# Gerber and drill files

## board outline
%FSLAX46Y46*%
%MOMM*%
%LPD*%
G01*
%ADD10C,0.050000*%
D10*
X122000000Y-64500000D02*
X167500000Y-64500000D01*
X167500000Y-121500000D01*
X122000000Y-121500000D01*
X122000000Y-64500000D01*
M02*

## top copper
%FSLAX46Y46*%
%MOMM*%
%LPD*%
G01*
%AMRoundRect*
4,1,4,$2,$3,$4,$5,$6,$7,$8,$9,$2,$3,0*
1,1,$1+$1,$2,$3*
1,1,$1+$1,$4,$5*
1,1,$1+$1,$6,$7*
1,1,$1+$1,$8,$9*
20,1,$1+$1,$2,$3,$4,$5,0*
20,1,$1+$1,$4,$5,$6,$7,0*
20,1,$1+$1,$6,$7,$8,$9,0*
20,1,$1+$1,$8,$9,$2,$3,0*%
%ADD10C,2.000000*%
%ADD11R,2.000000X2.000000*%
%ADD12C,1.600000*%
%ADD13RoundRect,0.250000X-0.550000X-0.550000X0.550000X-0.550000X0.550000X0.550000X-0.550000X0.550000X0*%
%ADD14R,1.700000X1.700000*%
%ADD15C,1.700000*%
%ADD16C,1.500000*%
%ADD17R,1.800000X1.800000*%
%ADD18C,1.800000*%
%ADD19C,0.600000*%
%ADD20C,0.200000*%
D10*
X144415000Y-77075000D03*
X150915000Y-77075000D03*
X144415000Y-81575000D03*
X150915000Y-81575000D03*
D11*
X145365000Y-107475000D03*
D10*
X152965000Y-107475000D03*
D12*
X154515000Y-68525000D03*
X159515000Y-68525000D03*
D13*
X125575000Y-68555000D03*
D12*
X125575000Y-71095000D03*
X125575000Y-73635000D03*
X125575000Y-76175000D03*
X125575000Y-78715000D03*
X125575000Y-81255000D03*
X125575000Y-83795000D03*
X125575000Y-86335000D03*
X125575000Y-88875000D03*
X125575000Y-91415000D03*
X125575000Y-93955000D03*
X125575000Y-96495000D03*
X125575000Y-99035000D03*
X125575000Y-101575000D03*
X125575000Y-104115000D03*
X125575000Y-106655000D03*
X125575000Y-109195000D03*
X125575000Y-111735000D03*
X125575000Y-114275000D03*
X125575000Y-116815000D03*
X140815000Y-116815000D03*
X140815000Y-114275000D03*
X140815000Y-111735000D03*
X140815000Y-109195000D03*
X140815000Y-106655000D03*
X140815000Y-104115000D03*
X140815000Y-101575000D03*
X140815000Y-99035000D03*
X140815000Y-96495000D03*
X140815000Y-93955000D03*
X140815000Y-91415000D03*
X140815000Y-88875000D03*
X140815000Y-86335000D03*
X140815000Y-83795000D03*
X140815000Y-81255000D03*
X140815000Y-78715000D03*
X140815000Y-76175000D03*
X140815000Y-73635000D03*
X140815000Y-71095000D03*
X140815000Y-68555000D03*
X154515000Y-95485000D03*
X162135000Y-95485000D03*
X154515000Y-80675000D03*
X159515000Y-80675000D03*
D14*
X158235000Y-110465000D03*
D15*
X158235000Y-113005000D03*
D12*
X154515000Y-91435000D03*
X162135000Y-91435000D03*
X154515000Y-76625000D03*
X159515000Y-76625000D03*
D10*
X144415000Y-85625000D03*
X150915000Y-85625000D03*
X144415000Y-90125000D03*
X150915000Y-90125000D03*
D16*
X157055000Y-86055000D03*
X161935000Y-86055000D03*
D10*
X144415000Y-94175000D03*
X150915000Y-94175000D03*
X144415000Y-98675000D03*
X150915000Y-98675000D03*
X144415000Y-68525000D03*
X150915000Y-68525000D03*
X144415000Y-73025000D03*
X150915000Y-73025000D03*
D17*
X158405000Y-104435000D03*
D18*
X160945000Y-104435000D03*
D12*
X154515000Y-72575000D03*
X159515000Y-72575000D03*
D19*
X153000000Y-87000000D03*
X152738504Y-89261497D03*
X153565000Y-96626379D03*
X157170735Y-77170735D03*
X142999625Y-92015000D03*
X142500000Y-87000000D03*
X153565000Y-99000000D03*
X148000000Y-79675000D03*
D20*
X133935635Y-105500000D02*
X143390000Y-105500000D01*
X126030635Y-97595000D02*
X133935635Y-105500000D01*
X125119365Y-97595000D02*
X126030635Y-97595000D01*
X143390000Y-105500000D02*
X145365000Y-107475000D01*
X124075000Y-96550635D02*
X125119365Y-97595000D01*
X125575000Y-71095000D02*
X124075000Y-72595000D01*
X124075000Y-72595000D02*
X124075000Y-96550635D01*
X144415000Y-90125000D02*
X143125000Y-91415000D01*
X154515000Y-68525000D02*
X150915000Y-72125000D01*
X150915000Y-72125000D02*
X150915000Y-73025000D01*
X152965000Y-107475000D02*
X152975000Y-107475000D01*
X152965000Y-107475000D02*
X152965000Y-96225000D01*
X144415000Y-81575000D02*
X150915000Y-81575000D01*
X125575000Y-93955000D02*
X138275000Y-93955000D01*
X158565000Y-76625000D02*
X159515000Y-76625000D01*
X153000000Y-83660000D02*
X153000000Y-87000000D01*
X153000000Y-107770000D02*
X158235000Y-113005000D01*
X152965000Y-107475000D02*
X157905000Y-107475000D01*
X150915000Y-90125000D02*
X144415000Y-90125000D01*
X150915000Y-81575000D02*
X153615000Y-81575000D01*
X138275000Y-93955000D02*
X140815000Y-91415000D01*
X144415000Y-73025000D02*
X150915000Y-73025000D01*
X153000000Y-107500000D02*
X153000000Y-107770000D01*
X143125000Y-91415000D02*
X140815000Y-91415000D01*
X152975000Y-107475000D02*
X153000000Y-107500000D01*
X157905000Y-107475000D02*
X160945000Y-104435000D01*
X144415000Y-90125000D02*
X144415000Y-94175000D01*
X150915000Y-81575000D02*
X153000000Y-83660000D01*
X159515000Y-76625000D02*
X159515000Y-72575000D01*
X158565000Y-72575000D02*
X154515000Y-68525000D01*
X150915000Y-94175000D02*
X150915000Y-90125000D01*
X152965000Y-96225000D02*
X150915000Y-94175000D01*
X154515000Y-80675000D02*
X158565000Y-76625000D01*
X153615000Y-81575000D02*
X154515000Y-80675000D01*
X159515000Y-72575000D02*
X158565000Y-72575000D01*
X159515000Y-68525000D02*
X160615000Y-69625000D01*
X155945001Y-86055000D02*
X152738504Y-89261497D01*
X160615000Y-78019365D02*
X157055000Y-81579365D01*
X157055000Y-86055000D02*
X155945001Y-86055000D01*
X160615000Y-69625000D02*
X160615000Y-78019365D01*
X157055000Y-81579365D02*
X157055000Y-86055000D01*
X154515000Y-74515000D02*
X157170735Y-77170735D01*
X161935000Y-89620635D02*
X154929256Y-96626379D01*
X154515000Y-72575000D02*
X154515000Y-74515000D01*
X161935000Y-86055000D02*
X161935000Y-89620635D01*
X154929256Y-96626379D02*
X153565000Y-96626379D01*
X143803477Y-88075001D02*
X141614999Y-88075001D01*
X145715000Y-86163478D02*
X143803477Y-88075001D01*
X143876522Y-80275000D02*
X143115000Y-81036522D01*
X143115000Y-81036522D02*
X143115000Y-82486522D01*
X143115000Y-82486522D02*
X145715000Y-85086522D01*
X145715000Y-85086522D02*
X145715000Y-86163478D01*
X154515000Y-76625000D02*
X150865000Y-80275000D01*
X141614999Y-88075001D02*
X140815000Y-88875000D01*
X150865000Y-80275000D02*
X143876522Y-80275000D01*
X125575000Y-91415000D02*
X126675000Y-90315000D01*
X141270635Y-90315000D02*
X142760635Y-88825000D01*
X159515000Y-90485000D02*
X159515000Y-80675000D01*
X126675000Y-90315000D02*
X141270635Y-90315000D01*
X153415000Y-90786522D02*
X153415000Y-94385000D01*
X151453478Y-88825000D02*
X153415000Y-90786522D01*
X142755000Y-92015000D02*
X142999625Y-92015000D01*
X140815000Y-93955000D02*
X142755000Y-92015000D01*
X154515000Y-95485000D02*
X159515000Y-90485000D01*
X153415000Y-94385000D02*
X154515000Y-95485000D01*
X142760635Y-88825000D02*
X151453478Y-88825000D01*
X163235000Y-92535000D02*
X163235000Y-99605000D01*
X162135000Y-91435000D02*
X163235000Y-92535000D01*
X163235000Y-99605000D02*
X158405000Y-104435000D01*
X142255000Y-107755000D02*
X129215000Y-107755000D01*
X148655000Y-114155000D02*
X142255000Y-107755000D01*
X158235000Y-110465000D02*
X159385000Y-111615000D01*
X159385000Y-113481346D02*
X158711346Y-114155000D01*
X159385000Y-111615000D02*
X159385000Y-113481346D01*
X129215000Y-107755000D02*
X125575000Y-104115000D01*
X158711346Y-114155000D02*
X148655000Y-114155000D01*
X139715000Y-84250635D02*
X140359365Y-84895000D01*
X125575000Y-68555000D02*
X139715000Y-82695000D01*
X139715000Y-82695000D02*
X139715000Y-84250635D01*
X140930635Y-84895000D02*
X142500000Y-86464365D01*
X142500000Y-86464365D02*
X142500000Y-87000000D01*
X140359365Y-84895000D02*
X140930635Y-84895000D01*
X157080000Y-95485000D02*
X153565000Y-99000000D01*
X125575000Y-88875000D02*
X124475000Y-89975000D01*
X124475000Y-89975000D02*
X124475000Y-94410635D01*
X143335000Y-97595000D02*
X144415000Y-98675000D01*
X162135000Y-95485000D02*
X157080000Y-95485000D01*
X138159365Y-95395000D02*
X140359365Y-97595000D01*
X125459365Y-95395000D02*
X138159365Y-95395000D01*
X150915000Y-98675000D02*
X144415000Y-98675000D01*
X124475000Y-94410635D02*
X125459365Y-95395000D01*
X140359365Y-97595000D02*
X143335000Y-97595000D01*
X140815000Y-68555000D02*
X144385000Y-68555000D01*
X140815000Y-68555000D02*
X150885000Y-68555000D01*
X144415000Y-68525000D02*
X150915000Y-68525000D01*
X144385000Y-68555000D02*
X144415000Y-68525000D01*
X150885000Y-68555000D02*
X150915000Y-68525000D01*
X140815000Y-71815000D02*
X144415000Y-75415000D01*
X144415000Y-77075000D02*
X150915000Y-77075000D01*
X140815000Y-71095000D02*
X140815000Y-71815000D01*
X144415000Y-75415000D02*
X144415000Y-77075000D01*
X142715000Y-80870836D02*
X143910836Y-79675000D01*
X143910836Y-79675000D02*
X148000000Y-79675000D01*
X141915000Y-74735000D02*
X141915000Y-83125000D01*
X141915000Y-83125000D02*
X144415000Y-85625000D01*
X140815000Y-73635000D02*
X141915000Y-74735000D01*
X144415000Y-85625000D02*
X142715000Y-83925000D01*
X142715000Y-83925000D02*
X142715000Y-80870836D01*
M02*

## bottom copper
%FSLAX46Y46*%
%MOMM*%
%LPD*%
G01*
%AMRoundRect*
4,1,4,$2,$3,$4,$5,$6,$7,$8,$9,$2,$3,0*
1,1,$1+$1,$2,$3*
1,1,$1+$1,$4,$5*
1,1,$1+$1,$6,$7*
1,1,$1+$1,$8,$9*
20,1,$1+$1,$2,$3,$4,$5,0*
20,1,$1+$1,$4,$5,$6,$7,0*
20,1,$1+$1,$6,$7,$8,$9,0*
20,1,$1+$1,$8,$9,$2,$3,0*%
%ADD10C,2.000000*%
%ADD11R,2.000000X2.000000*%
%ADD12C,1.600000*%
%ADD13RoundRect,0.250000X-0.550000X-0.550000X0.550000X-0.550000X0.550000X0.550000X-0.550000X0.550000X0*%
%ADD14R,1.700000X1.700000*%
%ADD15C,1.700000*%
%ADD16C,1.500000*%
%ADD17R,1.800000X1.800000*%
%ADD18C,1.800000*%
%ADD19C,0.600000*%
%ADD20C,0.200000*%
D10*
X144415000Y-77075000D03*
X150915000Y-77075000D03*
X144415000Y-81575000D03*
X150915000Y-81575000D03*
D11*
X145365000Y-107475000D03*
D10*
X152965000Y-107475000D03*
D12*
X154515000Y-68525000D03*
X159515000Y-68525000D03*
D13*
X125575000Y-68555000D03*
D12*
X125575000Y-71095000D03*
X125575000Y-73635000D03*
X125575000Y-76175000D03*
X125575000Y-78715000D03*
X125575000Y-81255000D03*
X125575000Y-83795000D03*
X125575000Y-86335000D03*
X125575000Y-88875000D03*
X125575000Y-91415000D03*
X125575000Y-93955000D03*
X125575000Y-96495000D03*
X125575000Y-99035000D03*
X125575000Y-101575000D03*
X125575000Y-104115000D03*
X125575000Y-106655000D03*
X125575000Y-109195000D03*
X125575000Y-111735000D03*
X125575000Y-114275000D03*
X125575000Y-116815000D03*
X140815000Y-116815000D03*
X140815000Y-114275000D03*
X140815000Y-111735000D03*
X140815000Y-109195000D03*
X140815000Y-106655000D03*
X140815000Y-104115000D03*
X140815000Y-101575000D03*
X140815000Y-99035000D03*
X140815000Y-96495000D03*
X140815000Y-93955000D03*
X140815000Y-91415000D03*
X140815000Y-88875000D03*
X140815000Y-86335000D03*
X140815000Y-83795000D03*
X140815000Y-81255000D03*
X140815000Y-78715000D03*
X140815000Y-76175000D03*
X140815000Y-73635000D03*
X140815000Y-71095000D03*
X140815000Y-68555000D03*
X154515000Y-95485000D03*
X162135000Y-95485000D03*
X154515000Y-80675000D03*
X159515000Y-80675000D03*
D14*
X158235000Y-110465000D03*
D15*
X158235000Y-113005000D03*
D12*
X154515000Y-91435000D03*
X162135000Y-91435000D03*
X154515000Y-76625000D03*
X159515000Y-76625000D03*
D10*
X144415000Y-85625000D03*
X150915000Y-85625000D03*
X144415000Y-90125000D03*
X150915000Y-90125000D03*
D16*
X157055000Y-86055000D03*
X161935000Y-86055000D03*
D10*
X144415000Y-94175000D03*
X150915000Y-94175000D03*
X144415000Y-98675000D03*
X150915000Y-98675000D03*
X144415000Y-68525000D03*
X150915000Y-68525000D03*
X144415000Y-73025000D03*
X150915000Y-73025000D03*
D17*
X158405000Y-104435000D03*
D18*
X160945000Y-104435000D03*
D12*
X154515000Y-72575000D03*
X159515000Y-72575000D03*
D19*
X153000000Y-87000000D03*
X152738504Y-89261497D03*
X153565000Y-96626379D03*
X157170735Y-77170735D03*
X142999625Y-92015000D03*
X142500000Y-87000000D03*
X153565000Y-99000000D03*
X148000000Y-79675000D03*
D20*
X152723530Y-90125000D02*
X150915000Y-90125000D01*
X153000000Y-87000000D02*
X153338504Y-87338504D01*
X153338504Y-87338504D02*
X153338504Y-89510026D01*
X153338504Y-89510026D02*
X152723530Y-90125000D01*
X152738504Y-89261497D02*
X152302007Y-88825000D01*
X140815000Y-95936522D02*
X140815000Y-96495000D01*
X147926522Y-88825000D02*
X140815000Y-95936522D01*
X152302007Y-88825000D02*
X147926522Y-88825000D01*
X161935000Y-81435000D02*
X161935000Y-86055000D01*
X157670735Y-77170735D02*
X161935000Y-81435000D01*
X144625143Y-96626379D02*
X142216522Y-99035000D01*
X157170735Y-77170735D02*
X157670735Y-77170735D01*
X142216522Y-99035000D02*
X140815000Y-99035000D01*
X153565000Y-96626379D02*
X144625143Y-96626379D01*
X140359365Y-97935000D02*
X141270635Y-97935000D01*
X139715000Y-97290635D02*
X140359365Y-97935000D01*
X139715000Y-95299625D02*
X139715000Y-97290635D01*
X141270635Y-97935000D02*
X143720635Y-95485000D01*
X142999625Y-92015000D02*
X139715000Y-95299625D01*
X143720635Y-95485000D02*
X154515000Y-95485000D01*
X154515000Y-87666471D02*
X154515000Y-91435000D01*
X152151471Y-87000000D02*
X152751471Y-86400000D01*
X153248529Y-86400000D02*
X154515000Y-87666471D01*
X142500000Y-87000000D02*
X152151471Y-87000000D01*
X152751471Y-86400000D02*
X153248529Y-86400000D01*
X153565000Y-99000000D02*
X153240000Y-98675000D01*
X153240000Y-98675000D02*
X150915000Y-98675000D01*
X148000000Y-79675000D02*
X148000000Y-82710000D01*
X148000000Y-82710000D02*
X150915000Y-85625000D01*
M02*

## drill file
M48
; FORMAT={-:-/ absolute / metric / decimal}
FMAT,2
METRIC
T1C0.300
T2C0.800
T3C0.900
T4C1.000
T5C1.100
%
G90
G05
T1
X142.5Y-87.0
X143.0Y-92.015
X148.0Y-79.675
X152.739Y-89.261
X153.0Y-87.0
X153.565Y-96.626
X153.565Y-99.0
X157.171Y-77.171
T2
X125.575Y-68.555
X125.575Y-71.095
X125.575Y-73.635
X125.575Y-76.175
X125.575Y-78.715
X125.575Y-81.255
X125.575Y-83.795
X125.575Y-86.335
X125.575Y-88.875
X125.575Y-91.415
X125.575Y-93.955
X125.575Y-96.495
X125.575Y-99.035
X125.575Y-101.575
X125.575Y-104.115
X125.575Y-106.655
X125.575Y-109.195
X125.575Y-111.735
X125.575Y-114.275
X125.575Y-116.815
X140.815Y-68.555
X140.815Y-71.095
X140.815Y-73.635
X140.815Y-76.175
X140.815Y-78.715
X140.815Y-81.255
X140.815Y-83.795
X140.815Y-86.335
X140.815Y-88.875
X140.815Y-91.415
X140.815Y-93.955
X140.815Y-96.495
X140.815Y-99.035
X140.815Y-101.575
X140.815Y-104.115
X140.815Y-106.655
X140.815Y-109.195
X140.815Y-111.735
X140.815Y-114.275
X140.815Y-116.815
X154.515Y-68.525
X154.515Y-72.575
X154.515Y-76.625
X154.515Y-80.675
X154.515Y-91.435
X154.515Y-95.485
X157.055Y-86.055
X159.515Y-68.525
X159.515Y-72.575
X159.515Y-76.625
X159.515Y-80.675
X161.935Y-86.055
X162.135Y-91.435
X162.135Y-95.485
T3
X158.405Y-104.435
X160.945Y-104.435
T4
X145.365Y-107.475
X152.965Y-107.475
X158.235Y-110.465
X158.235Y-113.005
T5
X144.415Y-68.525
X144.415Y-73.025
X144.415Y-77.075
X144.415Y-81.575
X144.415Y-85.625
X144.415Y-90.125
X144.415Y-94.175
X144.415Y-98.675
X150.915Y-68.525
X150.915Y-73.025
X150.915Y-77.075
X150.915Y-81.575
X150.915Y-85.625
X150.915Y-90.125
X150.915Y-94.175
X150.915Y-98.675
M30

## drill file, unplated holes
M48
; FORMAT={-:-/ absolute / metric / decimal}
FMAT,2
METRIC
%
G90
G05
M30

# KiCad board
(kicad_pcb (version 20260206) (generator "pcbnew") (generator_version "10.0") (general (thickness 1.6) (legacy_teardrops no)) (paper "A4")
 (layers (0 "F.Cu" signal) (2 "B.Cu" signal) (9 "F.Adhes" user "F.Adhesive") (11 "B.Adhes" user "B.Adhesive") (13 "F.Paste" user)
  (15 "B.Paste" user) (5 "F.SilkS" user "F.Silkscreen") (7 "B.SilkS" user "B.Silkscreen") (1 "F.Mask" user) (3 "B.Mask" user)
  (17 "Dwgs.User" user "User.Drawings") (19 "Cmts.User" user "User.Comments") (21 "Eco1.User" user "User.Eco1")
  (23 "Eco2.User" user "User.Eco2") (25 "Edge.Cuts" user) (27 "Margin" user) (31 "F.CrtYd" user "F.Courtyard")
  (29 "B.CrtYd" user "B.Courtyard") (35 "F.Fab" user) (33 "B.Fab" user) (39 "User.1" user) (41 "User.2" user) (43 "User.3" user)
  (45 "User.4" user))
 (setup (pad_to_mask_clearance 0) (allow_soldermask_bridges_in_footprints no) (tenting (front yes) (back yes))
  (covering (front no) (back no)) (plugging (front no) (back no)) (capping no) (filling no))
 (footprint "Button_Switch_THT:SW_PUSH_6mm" (layer "F.Cu") (at 144.415 77.075)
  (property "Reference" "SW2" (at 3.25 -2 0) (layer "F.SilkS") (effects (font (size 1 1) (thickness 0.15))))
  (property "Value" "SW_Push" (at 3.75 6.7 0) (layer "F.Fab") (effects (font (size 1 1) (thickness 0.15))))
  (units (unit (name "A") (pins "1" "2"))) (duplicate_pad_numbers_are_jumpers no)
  (pad "1" thru_hole circle (at 0 0 90) (size 2 2) (drill 1.1) (layers "*.Cu" "*.Mask") (remove_unused_layers no) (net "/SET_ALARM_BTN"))
  (pad "1" thru_hole circle (at 6.5 0 90) (size 2 2) (drill 1.1) (layers "*.Cu" "*.Mask") (remove_unused_layers no) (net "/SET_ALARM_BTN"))
  (pad "2" thru_hole circle (at 0 4.5 90) (size 2 2) (drill 1.1) (layers "*.Cu" "*.Mask") (remove_unused_layers no) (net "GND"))
  (pad "2" thru_hole circle (at 6.5 4.5 90) (size 2 2) (drill 1.1) (layers "*.Cu" "*.Mask") (remove_unused_layers no) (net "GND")))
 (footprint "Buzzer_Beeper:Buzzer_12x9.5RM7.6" (layer "F.Cu") (at 145.365 107.475)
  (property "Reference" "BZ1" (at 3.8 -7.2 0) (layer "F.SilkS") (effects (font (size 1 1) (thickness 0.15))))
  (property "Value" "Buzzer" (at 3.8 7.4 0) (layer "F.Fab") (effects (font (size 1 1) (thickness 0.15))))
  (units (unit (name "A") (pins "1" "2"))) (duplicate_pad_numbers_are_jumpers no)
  (pad "1" thru_hole rect (at 0 0) (size 2 2) (drill 1) (layers "*.Cu" "*.Mask") (remove_unused_layers no) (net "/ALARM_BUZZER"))
  (pad "2" thru_hole circle (at 7.6 0) (size 2 2) (drill 1) (layers "*.Cu" "*.Mask") (remove_unused_layers no) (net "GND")))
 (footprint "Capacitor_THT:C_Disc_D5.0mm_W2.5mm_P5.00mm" (layer "F.Cu") (at 154.515 68.525)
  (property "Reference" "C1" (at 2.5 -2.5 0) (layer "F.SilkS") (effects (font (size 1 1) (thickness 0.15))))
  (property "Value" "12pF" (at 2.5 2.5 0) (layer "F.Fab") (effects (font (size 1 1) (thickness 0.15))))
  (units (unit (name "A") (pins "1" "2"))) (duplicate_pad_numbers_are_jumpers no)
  (pad "1" thru_hole circle (at 0 0) (size 1.6 1.6) (drill 0.8) (layers "*.Cu" "*.Mask") (remove_unused_layers no) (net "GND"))
  (pad "2" thru_hole circle (at 5 0) (size 1.6 1.6) (drill 0.8) (layers "*.Cu" "*.Mask") (remove_unused_layers no) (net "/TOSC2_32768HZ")))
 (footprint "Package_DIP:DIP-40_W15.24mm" (layer "F.Cu") (at 125.575 68.555)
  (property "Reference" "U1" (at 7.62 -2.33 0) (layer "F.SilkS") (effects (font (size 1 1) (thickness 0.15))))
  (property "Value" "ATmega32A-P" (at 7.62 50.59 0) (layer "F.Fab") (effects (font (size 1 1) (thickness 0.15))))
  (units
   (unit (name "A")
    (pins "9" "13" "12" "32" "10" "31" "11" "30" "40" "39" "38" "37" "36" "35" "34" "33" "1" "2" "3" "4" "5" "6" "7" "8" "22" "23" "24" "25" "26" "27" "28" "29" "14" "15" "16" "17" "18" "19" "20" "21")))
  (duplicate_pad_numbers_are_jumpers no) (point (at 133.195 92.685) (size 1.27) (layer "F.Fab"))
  (pad "1" thru_hole roundrect (at 0 0) (size 1.6 1.6) (drill 0.8) (layers "*.Cu" "*.Mask") (remove_unused_layers no)
   (roundrect_rratio 0.15625) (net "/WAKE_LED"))
  (pad "2" thru_hole circle (at 0 2.54) (size 1.6 1.6) (drill 0.8) (layers "*.Cu" "*.Mask") (remove_unused_layers no) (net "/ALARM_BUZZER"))
  (pad "3" thru_hole circle (at 0 5.08) (size 1.6 1.6) (drill 0.8) (layers "*.Cu" "*.Mask") (remove_unused_layers no)
   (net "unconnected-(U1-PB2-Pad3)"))
  (pad "4" thru_hole circle (at 0 7.62) (size 1.6 1.6) (drill 0.8) (layers "*.Cu" "*.Mask") (remove_unused_layers no)
   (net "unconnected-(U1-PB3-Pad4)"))
  (pad "5" thru_hole circle (at 0 10.16) (size 1.6 1.6) (drill 0.8) (layers "*.Cu" "*.Mask") (remove_unused_layers no)
   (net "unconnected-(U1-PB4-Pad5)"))
  (pad "6" thru_hole circle (at 0 12.7) (size 1.6 1.6) (drill 0.8) (layers "*.Cu" "*.Mask") (remove_unused_layers no)
   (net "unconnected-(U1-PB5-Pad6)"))
  (pad "7" thru_hole circle (at 0 15.24) (size 1.6 1.6) (drill 0.8) (layers "*.Cu" "*.Mask") (remove_unused_layers no)
   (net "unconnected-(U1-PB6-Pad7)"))
  (pad "8" thru_hole circle (at 0 17.78) (size 1.6 1.6) (drill 0.8) (layers "*.Cu" "*.Mask") (remove_unused_layers no)
   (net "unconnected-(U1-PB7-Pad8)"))
  (pad "9" thru_hole circle (at 0 20.32) (size 1.6 1.6) (drill 0.8) (layers "*.Cu" "*.Mask") (remove_unused_layers no)
   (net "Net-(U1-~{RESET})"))
  (pad "10" thru_hole circle (at 0 22.86) (size 1.6 1.6) (drill 0.8) (layers "*.Cu" "*.Mask") (remove_unused_layers no) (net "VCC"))
  (pad "11" thru_hole circle (at 0 25.4) (size 1.6 1.6) (drill 0.8) (layers "*.Cu" "*.Mask") (remove_unused_layers no) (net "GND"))
  (pad "12" thru_hole circle (at 0 27.94) (size 1.6 1.6) (drill 0.8) (layers "*.Cu" "*.Mask") (remove_unused_layers no)
   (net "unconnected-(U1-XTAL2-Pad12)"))
  (pad "13" thru_hole circle (at 0 30.48) (size 1.6 1.6) (drill 0.8) (layers "*.Cu" "*.Mask") (remove_unused_layers no)
   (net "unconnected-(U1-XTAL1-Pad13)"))
  (pad "14" thru_hole circle (at 0 33.02) (size 1.6 1.6) (drill 0.8) (layers "*.Cu" "*.Mask") (remove_unused_layers no)
   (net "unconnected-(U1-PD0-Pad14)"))
  (pad "15" thru_hole circle (at 0 35.56) (size 1.6 1.6) (drill 0.8) (layers "*.Cu" "*.Mask") (remove_unused_layers no)
   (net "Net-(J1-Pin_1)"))
  (pad "16" thru_hole circle (at 0 38.1) (size 1.6 1.6) (drill 0.8) (layers "*.Cu" "*.Mask") (remove_unused_layers no)
   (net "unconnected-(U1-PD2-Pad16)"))
  (pad "17" thru_hole circle (at 0 40.64) (size 1.6 1.6) (drill 0.8) (layers "*.Cu" "*.Mask") (remove_unused_layers no)
   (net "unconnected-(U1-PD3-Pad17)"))
  (pad "18" thru_hole circle (at 0 43.18) (size 1.6 1.6) (drill 0.8) (layers "*.Cu" "*.Mask") (remove_unused_layers no)
   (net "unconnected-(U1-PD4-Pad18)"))
  (pad "19" thru_hole circle (at 0 45.72) (size 1.6 1.6) (drill 0.8) (layers "*.Cu" "*.Mask") (remove_unused_layers no)
   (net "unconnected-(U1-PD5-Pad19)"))
  (pad "20" thru_hole circle (at 0 48.26) (size 1.6 1.6) (drill 0.8) (layers "*.Cu" "*.Mask") (remove_unused_layers no)
   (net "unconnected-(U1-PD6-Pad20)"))
  (pad "21" thru_hole circle (at 15.24 48.26) (size 1.6 1.6) (drill 0.8) (layers "*.Cu" "*.Mask") (remove_unused_layers no)
   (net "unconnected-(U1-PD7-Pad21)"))
  (pad "22" thru_hole circle (at 15.24 45.72) (size 1.6 1.6) (drill 0.8) (layers "*.Cu" "*.Mask") (remove_unused_layers no)
   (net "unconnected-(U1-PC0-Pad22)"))
  (pad "23" thru_hole circle (at 15.24 43.18) (size 1.6 1.6) (drill 0.8) (layers "*.Cu" "*.Mask") (remove_unused_layers no)
   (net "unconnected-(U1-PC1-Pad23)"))
  (pad "24" thru_hole circle (at 15.24 40.64) (size 1.6 1.6) (drill 0.8) (layers "*.Cu" "*.Mask") (remove_unused_layers no)
   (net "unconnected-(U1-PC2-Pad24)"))
  (pad "25" thru_hole circle (at 15.24 38.1) (size 1.6 1.6) (drill 0.8) (layers "*.Cu" "*.Mask") (remove_unused_layers no)
   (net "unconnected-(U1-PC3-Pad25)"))
  (pad "26" thru_hole circle (at 15.24 35.56) (size 1.6 1.6) (drill 0.8) (layers "*.Cu" "*.Mask") (remove_unused_layers no)
   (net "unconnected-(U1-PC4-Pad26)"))
  (pad "27" thru_hole circle (at 15.24 33.02) (size 1.6 1.6) (drill 0.8) (layers "*.Cu" "*.Mask") (remove_unused_layers no)
   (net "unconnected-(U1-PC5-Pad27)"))
  (pad "28" thru_hole circle (at 15.24 30.48) (size 1.6 1.6) (drill 0.8) (layers "*.Cu" "*.Mask") (remove_unused_layers no)
   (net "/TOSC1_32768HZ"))
  (pad "29" thru_hole circle (at 15.24 27.94) (size 1.6 1.6) (drill 0.8) (layers "*.Cu" "*.Mask") (remove_unused_layers no)
   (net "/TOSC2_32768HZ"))
  (pad "30" thru_hole circle (at 15.24 25.4) (size 1.6 1.6) (drill 0.8) (layers "*.Cu" "*.Mask") (remove_unused_layers no) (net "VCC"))
  (pad "31" thru_hole circle (at 15.24 22.86) (size 1.6 1.6) (drill 0.8) (layers "*.Cu" "*.Mask") (remove_unused_layers no) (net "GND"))
  (pad "32" thru_hole circle (at 15.24 20.32) (size 1.6 1.6) (drill 0.8) (layers "*.Cu" "*.Mask") (remove_unused_layers no)
   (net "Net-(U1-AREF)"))
  (pad "33" thru_hole circle (at 15.24 17.78) (size 1.6 1.6) (drill 0.8) (layers "*.Cu" "*.Mask") (remove_unused_layers no)
   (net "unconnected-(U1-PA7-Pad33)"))
  (pad "34" thru_hole circle (at 15.24 15.24) (size 1.6 1.6) (drill 0.8) (layers "*.Cu" "*.Mask") (remove_unused_layers no)
   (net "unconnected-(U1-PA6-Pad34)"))
  (pad "35" thru_hole circle (at 15.24 12.7) (size 1.6 1.6) (drill 0.8) (layers "*.Cu" "*.Mask") (remove_unused_layers no)
   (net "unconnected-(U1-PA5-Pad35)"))
  (pad "36" thru_hole circle (at 15.24 10.16) (size 1.6 1.6) (drill 0.8) (layers "*.Cu" "*.Mask") (remove_unused_layers no)
   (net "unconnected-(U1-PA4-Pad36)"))
  (pad "37" thru_hole circle (at 15.24 7.62) (size 1.6 1.6) (drill 0.8) (layers "*.Cu" "*.Mask") (remove_unused_layers no)
   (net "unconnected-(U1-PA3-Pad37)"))
  (pad "38" thru_hole circle (at 15.24 5.08) (size 1.6 1.6) (drill 0.8) (layers "*.Cu" "*.Mask") (remove_unused_layers no)
   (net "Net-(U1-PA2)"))
  (pad "39" thru_hole circle (at 15.24 2.54) (size 1.6 1.6) (drill 0.8) (layers "*.Cu" "*.Mask") (remove_unused_layers no)
   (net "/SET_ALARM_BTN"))
  (pad "40" thru_hole circle (at 15.24 0) (size 1.6 1.6) (drill 0.8) (layers "*.Cu" "*.Mask") (remove_unused_layers no) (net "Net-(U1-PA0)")))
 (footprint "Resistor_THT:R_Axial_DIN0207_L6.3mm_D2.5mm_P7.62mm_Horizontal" (layer "F.Cu") (at 154.515 95.485)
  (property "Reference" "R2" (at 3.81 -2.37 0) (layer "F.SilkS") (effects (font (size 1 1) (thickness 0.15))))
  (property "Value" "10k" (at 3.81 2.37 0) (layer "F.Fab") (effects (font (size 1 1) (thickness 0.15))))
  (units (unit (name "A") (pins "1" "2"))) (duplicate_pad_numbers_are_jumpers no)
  (pad "1" thru_hole circle (at 0 0) (size 1.6 1.6) (drill 0.8) (layers "*.Cu" "*.Mask") (remove_unused_layers no) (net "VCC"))
  (pad "2" thru_hole circle (at 7.62 0) (size 1.6 1.6) (drill 0.8) (layers "*.Cu" "*.Mask") (remove_unused_layers no)
   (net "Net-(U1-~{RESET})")))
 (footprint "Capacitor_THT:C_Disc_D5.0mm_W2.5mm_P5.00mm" (layer "F.Cu") (at 154.515 80.675)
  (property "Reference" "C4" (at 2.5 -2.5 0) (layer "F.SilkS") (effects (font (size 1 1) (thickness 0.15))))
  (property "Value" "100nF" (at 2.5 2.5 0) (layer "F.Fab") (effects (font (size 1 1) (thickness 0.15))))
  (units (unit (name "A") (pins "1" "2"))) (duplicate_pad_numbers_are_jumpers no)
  (pad "1" thru_hole circle (at 0 0) (size 1.6 1.6) (drill 0.8) (layers "*.Cu" "*.Mask") (remove_unused_layers no) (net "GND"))
  (pad "2" thru_hole circle (at 5 0) (size 1.6 1.6) (drill 0.8) (layers "*.Cu" "*.Mask") (remove_unused_layers no) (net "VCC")))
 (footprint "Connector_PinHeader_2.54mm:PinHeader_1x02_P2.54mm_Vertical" (layer "F.Cu") (at 158.235 110.465)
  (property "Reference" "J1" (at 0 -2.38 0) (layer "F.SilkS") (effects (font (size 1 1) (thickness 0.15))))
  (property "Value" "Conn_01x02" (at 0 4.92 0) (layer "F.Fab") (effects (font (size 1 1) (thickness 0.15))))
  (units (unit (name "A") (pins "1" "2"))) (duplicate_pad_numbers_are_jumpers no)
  (pad "1" thru_hole rect (at 0 0) (size 1.7 1.7) (drill 1) (layers "*.Cu" "*.Mask") (remove_unused_layers no) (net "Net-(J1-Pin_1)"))
  (pad "2" thru_hole circle (at 0 2.54) (size 1.7 1.7) (drill 1) (layers "*.Cu" "*.Mask") (remove_unused_layers no) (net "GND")))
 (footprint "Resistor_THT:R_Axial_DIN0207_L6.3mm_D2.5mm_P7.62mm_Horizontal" (layer "F.Cu") (at 154.515 91.435)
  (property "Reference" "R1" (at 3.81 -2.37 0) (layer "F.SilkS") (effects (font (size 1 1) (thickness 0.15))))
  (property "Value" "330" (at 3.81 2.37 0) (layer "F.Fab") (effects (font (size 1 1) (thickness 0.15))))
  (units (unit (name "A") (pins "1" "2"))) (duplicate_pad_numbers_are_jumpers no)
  (pad "1" thru_hole circle (at 0 0) (size 1.6 1.6) (drill 0.8) (layers "*.Cu" "*.Mask") (remove_unused_layers no) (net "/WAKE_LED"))
  (pad "2" thru_hole circle (at 7.62 0) (size 1.6 1.6) (drill 0.8) (layers "*.Cu" "*.Mask") (remove_unused_layers no) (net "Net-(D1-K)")))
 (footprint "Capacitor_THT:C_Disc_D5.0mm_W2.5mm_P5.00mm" (layer "F.Cu") (at 154.515 76.625)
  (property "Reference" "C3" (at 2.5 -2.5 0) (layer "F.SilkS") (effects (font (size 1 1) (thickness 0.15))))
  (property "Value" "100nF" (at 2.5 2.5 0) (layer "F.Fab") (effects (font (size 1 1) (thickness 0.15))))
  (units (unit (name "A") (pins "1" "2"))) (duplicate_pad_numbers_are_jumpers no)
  (pad "1" thru_hole circle (at 0 0) (size 1.6 1.6) (drill 0.8) (layers "*.Cu" "*.Mask") (remove_unused_layers no) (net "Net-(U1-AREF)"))
  (pad "2" thru_hole circle (at 5 0) (size 1.6 1.6) (drill 0.8) (layers "*.Cu" "*.Mask") (remove_unused_layers no) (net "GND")))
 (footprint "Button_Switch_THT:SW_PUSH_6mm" (layer "F.Cu") (at 144.415 85.625)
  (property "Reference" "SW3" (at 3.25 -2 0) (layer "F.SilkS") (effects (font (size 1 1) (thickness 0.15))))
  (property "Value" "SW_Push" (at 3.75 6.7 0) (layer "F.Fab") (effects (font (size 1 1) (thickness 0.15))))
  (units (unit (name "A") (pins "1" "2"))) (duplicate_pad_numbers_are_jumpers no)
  (pad "1" thru_hole circle (at 0 0 90) (size 2 2) (drill 1.1) (layers "*.Cu" "*.Mask") (remove_unused_layers no) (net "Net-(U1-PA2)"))
  (pad "1" thru_hole circle (at 6.5 0 90) (size 2 2) (drill 1.1) (layers "*.Cu" "*.Mask") (remove_unused_layers no) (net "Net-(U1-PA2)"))
  (pad "2" thru_hole circle (at 0 4.5 90) (size 2 2) (drill 1.1) (layers "*.Cu" "*.Mask") (remove_unused_layers no) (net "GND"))
  (pad "2" thru_hole circle (at 6.5 4.5 90) (size 2 2) (drill 1.1) (layers "*.Cu" "*.Mask") (remove_unused_layers no) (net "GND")))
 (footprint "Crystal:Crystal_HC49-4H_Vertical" (layer "F.Cu") (at 157.055 86.055)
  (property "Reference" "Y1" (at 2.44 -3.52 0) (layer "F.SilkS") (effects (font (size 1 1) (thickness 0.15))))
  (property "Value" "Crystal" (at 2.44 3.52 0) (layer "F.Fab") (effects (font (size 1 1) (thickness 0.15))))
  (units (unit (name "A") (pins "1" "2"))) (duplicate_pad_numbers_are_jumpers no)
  (pad "1" thru_hole circle (at 0 0) (size 1.5 1.5) (drill 0.8) (layers "*.Cu" "*.Mask") (remove_unused_layers no) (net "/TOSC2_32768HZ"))
  (pad "2" thru_hole circle (at 4.88 0) (size 1.5 1.5) (drill 0.8) (layers "*.Cu" "*.Mask") (remove_unused_layers no) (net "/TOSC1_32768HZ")))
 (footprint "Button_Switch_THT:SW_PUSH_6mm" (layer "F.Cu") (at 144.415 94.175)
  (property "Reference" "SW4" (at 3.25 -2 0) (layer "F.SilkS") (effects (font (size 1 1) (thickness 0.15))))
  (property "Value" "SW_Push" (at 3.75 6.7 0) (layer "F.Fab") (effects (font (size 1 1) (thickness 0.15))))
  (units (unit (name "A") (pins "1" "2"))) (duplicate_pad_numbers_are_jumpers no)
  (pad "1" thru_hole circle (at 0 0 90) (size 2 2) (drill 1.1) (layers "*.Cu" "*.Mask") (remove_unused_layers no) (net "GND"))
  (pad "1" thru_hole circle (at 6.5 0 90) (size 2 2) (drill 1.1) (layers "*.Cu" "*.Mask") (remove_unused_layers no) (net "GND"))
  (pad "2" thru_hole circle (at 0 4.5 90) (size 2 2) (drill 1.1) (layers "*.Cu" "*.Mask") (remove_unused_layers no)
   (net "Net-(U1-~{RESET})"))
  (pad "2" thru_hole circle (at 6.5 4.5 90) (size 2 2) (drill 1.1) (layers "*.Cu" "*.Mask") (remove_unused_layers no)
   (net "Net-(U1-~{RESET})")))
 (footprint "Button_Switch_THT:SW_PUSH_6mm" (layer "F.Cu") (at 144.415 68.525)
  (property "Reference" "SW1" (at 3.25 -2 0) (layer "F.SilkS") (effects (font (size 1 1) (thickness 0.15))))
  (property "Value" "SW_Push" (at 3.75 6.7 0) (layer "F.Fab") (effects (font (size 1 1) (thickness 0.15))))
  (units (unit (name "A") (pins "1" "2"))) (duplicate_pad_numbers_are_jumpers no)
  (pad "1" thru_hole circle (at 0 0 90) (size 2 2) (drill 1.1) (layers "*.Cu" "*.Mask") (remove_unused_layers no) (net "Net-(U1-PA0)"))
  (pad "1" thru_hole circle (at 6.5 0 90) (size 2 2) (drill 1.1) (layers "*.Cu" "*.Mask") (remove_unused_layers no) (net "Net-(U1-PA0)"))
  (pad "2" thru_hole circle (at 0 4.5 90) (size 2 2) (drill 1.1) (layers "*.Cu" "*.Mask") (remove_unused_layers no) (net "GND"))
  (pad "2" thru_hole circle (at 6.5 4.5 90) (size 2 2) (drill 1.1) (layers "*.Cu" "*.Mask") (remove_unused_layers no) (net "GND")))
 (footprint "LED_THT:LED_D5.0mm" (layer "F.Cu") (at 158.405 104.435)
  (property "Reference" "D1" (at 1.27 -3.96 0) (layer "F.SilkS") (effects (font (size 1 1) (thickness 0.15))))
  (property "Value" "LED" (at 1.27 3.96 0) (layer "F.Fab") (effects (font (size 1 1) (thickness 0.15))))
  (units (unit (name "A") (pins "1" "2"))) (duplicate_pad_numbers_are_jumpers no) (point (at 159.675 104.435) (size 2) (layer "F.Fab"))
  (pad "1" thru_hole rect (at 0 0) (size 1.8 1.8) (drill 0.9) (layers "*.Cu" "*.Mask") (remove_unused_layers no) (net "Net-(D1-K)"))
  (pad "2" thru_hole circle (at 2.54 0) (size 1.8 1.8) (drill 0.9) (layers "*.Cu" "*.Mask") (remove_unused_layers no) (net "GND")))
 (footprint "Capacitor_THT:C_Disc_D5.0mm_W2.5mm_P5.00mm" (layer "F.Cu") (at 154.515 72.575)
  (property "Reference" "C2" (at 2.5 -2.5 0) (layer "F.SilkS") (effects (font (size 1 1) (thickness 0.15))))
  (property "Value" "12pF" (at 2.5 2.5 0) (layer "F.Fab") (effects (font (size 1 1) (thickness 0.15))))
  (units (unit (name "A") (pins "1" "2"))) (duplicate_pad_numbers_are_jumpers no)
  (pad "1" thru_hole circle (at 0 0) (size 1.6 1.6) (drill 0.8) (layers "*.Cu" "*.Mask") (remove_unused_layers no) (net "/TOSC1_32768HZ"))
  (pad "2" thru_hole circle (at 5 0) (size 1.6 1.6) (drill 0.8) (layers "*.Cu" "*.Mask") (remove_unused_layers no) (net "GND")))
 (gr_rect (start 122 64.5) (end 167.5 121.5) (stroke (width 0.05) (type default)) (fill no) (layer "Edge.Cuts"))
 (segment (start 133.935635 105.5) (end 143.39 105.5) (width 0.2) (layer "F.Cu") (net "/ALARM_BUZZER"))
 (segment (start 126.030635 97.595) (end 133.935635 105.5) (width 0.2) (layer "F.Cu") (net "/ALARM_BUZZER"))
 (segment (start 125.119365 97.595) (end 126.030635 97.595) (width 0.2) (layer "F.Cu") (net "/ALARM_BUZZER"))
 (segment (start 143.39 105.5) (end 145.365 107.475) (width 0.2) (layer "F.Cu") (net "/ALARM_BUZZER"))
 (segment (start 124.075 96.550635) (end 125.119365 97.595) (width 0.2) (layer "F.Cu") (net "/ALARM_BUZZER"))
 (segment (start 125.575 71.095) (end 124.075 72.595) (width 0.2) (layer "F.Cu") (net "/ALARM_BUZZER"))
 (segment (start 124.075 72.595) (end 124.075 96.550635) (width 0.2) (layer "F.Cu") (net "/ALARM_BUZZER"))
 (segment (start 144.415 90.125) (end 143.125 91.415) (width 0.2) (layer "F.Cu") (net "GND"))
 (segment (start 154.515 68.525) (end 150.915 72.125) (width 0.2) (layer "F.Cu") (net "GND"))
 (segment (start 150.915 72.125) (end 150.915 73.025) (width 0.2) (layer "F.Cu") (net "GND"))
 (segment (start 152.965 107.475) (end 152.975 107.475) (width 0.2) (layer "F.Cu") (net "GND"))
 (segment (start 152.965 107.475) (end 152.965 96.225) (width 0.2) (layer "F.Cu") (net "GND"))
 (segment (start 144.415 81.575) (end 150.915 81.575) (width 0.2) (layer "F.Cu") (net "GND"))
 (segment (start 125.575 93.955) (end 138.275 93.955) (width 0.2) (layer "F.Cu") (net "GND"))
 (segment (start 158.565 76.625) (end 159.515 76.625) (width 0.2) (layer "F.Cu") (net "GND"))
 (segment (start 153 83.66) (end 153 87) (width 0.2) (layer "F.Cu") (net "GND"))
 (segment (start 153 107.77) (end 158.235 113.005) (width 0.2) (layer "F.Cu") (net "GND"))
 (segment (start 152.965 107.475) (end 157.905 107.475) (width 0.2) (layer "F.Cu") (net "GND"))
 (segment (start 150.915 90.125) (end 144.415 90.125) (width 0.2) (layer "F.Cu") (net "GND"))
 (segment (start 150.915 81.575) (end 153.615 81.575) (width 0.2) (layer "F.Cu") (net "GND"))
 (segment (start 138.275 93.955) (end 140.815 91.415) (width 0.2) (layer "F.Cu") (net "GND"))
 (segment (start 144.415 73.025) (end 150.915 73.025) (width 0.2) (layer "F.Cu") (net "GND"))
 (segment (start 153 107.5) (end 153 107.77) (width 0.2) (layer "F.Cu") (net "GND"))
 (segment (start 143.125 91.415) (end 140.815 91.415) (width 0.2) (layer "F.Cu") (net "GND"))
 (segment (start 152.975 107.475) (end 153 107.5) (width 0.2) (layer "F.Cu") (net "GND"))
 (segment (start 157.905 107.475) (end 160.945 104.435) (width 0.2) (layer "F.Cu") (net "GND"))
 (segment (start 144.415 90.125) (end 144.415 94.175) (width 0.2) (layer "F.Cu") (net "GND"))
 (segment (start 150.915 81.575) (end 153 83.66) (width 0.2) (layer "F.Cu") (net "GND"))
 (segment (start 159.515 76.625) (end 159.515 72.575) (width 0.2) (layer "F.Cu") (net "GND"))
 (segment (start 158.565 72.575) (end 154.515 68.525) (width 0.2) (layer "F.Cu") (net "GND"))
 (segment (start 150.915 94.175) (end 150.915 90.125) (width 0.2) (layer "F.Cu") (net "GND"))
 (segment (start 152.965 96.225) (end 150.915 94.175) (width 0.2) (layer "F.Cu") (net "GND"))
 (segment (start 154.515 80.675) (end 158.565 76.625) (width 0.2) (layer "F.Cu") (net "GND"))
 (segment (start 153.615 81.575) (end 154.515 80.675) (width 0.2) (layer "F.Cu") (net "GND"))
 (segment (start 159.515 72.575) (end 158.565 72.575) (width 0.2) (layer "F.Cu") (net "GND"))
 (via (at 153 87) (size 0.6) (drill 0.3) (layers "F.Cu" "B.Cu") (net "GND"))
 (segment (start 152.72353 90.125) (end 150.915 90.125) (width 0.2) (layer "B.Cu") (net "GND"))
 (segment (start 153 87) (end 153.338504 87.338504) (width 0.2) (layer "B.Cu") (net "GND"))
 (segment (start 153.338504 87.338504) (end 153.338504 89.510026) (width 0.2) (layer "B.Cu") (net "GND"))
 (segment (start 153.338504 89.510026) (end 152.72353 90.125) (width 0.2) (layer "B.Cu") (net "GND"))
 (segment (start 159.515 68.525) (end 160.615 69.625) (width 0.2) (layer "F.Cu") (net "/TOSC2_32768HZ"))
 (segment (start 155.945001 86.055) (end 152.738504 89.261497) (width 0.2) (layer "F.Cu") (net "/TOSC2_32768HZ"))
 (segment (start 160.615 78.019365) (end 157.055 81.579365) (width 0.2) (layer "F.Cu") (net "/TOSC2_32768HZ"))
 (segment (start 157.055 86.055) (end 155.945001 86.055) (width 0.2) (layer "F.Cu") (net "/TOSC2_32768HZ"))
 (segment (start 160.615 69.625) (end 160.615 78.019365) (width 0.2) (layer "F.Cu") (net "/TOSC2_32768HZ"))
 (segment (start 157.055 81.579365) (end 157.055 86.055) (width 0.2) (layer "F.Cu") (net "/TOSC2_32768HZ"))
 (via (at 152.738504 89.261497) (size 0.6) (drill 0.3) (layers "F.Cu" "B.Cu") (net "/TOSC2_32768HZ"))
 (segment (start 152.738504 89.261497) (end 152.302007 88.825) (width 0.2) (layer "B.Cu") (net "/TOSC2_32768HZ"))
 (segment (start 140.815 95.936522) (end 140.815 96.495) (width 0.2) (layer "B.Cu") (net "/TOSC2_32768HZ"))
 (segment (start 147.926522 88.825) (end 140.815 95.936522) (width 0.2) (layer "B.Cu") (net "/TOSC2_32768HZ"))
 (segment (start 152.302007 88.825) (end 147.926522 88.825) (width 0.2) (layer "B.Cu") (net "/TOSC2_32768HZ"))
 (segment (start 154.515 74.515) (end 157.170735 77.170735) (width 0.2) (layer "F.Cu") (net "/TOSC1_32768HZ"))
 (segment (start 161.935 89.620635) (end 154.929256 96.626379) (width 0.2) (layer "F.Cu") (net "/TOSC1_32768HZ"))
 (segment (start 154.515 72.575) (end 154.515 74.515) (width 0.2) (layer "F.Cu") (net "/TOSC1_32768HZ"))
 (segment (start 161.935 86.055) (end 161.935 89.620635) (width 0.2) (layer "F.Cu") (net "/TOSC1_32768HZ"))
 (segment (start 154.929256 96.626379) (end 153.565 96.626379) (width 0.2) (layer "F.Cu") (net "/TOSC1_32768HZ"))
 (via (at 153.565 96.626379) (size 0.6) (drill 0.3) (layers "F.Cu" "B.Cu") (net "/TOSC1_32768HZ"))
 (via (at 157.170735 77.170735) (size 0.6) (drill 0.3) (layers "F.Cu" "B.Cu") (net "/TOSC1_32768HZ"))
 (segment (start 161.935 81.435) (end 161.935 86.055) (width 0.2) (layer "B.Cu") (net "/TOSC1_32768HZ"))
 (segment (start 157.670735 77.170735) (end 161.935 81.435) (width 0.2) (layer "B.Cu") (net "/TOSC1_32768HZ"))
 (segment (start 144.625143 96.626379) (end 142.216522 99.035) (width 0.2) (layer "B.Cu") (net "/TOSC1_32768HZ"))
 (segment (start 157.170735 77.170735) (end 157.670735 77.170735) (width 0.2) (layer "B.Cu") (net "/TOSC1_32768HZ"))
 (segment (start 142.216522 99.035) (end 140.815 99.035) (width 0.2) (layer "B.Cu") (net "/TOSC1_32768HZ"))
 (segment (start 153.565 96.626379) (end 144.625143 96.626379) (width 0.2) (layer "B.Cu") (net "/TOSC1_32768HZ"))
 (segment (start 143.803477 88.075001) (end 141.614999 88.075001) (width 0.2) (layer "F.Cu") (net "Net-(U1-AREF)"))
 (segment (start 145.715 86.163478) (end 143.803477 88.075001) (width 0.2) (layer "F.Cu") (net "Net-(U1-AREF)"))
 (segment (start 143.876522 80.275) (end 143.115 81.036522) (width 0.2) (layer "F.Cu") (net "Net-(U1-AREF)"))
 (segment (start 143.115 81.036522) (end 143.115 82.486522) (width 0.2) (layer "F.Cu") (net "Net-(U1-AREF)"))
 (segment (start 143.115 82.486522) (end 145.715 85.086522) (width 0.2) (layer "F.Cu") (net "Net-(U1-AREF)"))
 (segment (start 145.715 85.086522) (end 145.715 86.163478) (width 0.2) (layer "F.Cu") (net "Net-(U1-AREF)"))
 (segment (start 154.515 76.625) (end 150.865 80.275) (width 0.2) (layer "F.Cu") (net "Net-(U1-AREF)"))
 (segment (start 141.614999 88.075001) (end 140.815 88.875) (width 0.2) (layer "F.Cu") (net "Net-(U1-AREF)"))
 (segment (start 150.865 80.275) (end 143.876522 80.275) (width 0.2) (layer "F.Cu") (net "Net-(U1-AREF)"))
 (segment (start 125.575 91.415) (end 126.675 90.315) (width 0.2) (layer "F.Cu") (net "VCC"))
 (segment (start 141.270635 90.315) (end 142.760635 88.825) (width 0.2) (layer "F.Cu") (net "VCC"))
 (segment (start 159.515 90.485) (end 159.515 80.675) (width 0.2) (layer "F.Cu") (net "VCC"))
 (segment (start 126.675 90.315) (end 141.270635 90.315) (width 0.2) (layer "F.Cu") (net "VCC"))
 (segment (start 153.415 90.786522) (end 153.415 94.385) (width 0.2) (layer "F.Cu") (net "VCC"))
 (segment (start 151.453478 88.825) (end 153.415 90.786522) (width 0.2) (layer "F.Cu") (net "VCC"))
 (segment (start 142.755 92.015) (end 142.999625 92.015) (width 0.2) (layer "F.Cu") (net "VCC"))
 (segment (start 140.815 93.955) (end 142.755 92.015) (width 0.2) (layer "F.Cu") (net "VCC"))
 (segment (start 154.515 95.485) (end 159.515 90.485) (width 0.2) (layer "F.Cu") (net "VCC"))
 (segment (start 153.415 94.385) (end 154.515 95.485) (width 0.2) (layer "F.Cu") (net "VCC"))
 (segment (start 142.760635 88.825) (end 151.453478 88.825) (width 0.2) (layer "F.Cu") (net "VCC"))
 (via (at 142.999625 92.015) (size 0.6) (drill 0.3) (layers "F.Cu" "B.Cu") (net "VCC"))
 (segment (start 140.359365 97.935) (end 141.270635 97.935) (width 0.2) (layer "B.Cu") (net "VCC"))
 (segment (start 139.715 97.290635) (end 140.359365 97.935) (width 0.2) (layer "B.Cu") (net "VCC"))
 (segment (start 139.715 95.299625) (end 139.715 97.290635) (width 0.2) (layer "B.Cu") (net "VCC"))
 (segment (start 141.270635 97.935) (end 143.720635 95.485) (width 0.2) (layer "B.Cu") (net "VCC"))
 (segment (start 142.999625 92.015) (end 139.715 95.299625) (width 0.2) (layer "B.Cu") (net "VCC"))
 (segment (start 143.720635 95.485) (end 154.515 95.485) (width 0.2) (layer "B.Cu") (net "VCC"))
 (segment (start 163.235 92.535) (end 163.235 99.605) (width 0.2) (layer "F.Cu") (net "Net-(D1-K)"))
 (segment (start 162.135 91.435) (end 163.235 92.535) (width 0.2) (layer "F.Cu") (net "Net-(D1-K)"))
 (segment (start 163.235 99.605) (end 158.405 104.435) (width 0.2) (layer "F.Cu") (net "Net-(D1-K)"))
 (segment (start 142.255 107.755) (end 129.215 107.755) (width 0.2) (layer "F.Cu") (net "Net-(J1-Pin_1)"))
 (segment (start 148.655 114.155) (end 142.255 107.755) (width 0.2) (layer "F.Cu") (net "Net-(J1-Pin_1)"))
 (segment (start 158.235 110.465) (end 159.385 111.615) (width 0.2) (layer "F.Cu") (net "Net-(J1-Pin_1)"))
 (segment (start 159.385 113.481346) (end 158.711346 114.155) (width 0.2) (layer "F.Cu") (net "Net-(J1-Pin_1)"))
 (segment (start 159.385 111.615) (end 159.385 113.481346) (width 0.2) (layer "F.Cu") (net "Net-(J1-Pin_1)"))
 (segment (start 129.215 107.755) (end 125.575 104.115) (width 0.2) (layer "F.Cu") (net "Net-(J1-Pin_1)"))
 (segment (start 158.711346 114.155) (end 148.655 114.155) (width 0.2) (layer "F.Cu") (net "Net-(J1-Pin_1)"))
 (segment (start 139.715 84.250635) (end 140.359365 84.895) (width 0.2) (layer "F.Cu") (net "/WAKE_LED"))
 (segment (start 125.575 68.555) (end 139.715 82.695) (width 0.2) (layer "F.Cu") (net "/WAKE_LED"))
 (segment (start 139.715 82.695) (end 139.715 84.250635) (width 0.2) (layer "F.Cu") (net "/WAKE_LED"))
 (segment (start 140.930635 84.895) (end 142.5 86.464365) (width 0.2) (layer "F.Cu") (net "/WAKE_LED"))
 (segment (start 142.5 86.464365) (end 142.5 87) (width 0.2) (layer "F.Cu") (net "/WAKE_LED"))
 (segment (start 140.359365 84.895) (end 140.930635 84.895) (width 0.2) (layer "F.Cu") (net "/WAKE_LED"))
 (via (at 142.5 87) (size 0.6) (drill 0.3) (layers "F.Cu" "B.Cu") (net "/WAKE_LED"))
 (segment (start 154.515 87.666471) (end 154.515 91.435) (width 0.2) (layer "B.Cu") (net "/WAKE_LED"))
 (segment (start 152.151471 87) (end 152.751471 86.4) (width 0.2) (layer "B.Cu") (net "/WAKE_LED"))
 (segment (start 153.248529 86.4) (end 154.515 87.666471) (width 0.2) (layer "B.Cu") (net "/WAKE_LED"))
 (segment (start 142.5 87) (end 152.151471 87) (width 0.2) (layer "B.Cu") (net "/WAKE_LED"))
 (segment (start 152.751471 86.4) (end 153.248529 86.4) (width 0.2) (layer "B.Cu") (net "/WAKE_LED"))
 (segment (start 157.08 95.485) (end 153.565 99) (width 0.2) (layer "F.Cu") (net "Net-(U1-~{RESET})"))
 (segment (start 125.575 88.875) (end 124.475 89.975) (width 0.2) (layer "F.Cu") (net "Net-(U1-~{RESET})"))
 (segment (start 124.475 89.975) (end 124.475 94.410635) (width 0.2) (layer "F.Cu") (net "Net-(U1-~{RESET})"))
 (segment (start 143.335 97.595) (end 144.415 98.675) (width 0.2) (layer "F.Cu") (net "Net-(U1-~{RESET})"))
 (segment (start 162.135 95.485) (end 157.08 95.485) (width 0.2) (layer "F.Cu") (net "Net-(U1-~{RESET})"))
 (segment (start 138.159365 95.395) (end 140.359365 97.595) (width 0.2) (layer "F.Cu") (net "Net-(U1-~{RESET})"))
 (segment (start 125.459365 95.395) (end 138.159365 95.395) (width 0.2) (layer "F.Cu") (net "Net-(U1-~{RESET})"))
 (segment (start 150.915 98.675) (end 144.415 98.675) (width 0.2) (layer "F.Cu") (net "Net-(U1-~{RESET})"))
 (segment (start 124.475 94.410635) (end 125.459365 95.395) (width 0.2) (layer "F.Cu") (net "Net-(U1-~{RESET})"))
 (segment (start 140.359365 97.595) (end 143.335 97.595) (width 0.2) (layer "F.Cu") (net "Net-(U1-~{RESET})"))
 (via (at 153.565 99) (size 0.6) (drill 0.3) (layers "F.Cu" "B.Cu") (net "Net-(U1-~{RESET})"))
 (segment (start 153.565 99) (end 153.24 98.675) (width 0.2) (layer "B.Cu") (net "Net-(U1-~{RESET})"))
 (segment (start 153.24 98.675) (end 150.915 98.675) (width 0.2) (layer "B.Cu") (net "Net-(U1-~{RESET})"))
 (segment (start 140.815 68.555) (end 144.385 68.555) (width 0.2) (layer "F.Cu") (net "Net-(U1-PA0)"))
 (segment (start 140.815 68.555) (end 150.885 68.555) (width 0.2) (layer "F.Cu") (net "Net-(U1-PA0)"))
 (segment (start 144.415 68.525) (end 150.915 68.525) (width 0.2) (layer "F.Cu") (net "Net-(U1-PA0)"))
 (segment (start 144.385 68.555) (end 144.415 68.525) (width 0.2) (layer "F.Cu") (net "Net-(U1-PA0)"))
 (segment (start 150.885 68.555) (end 150.915 68.525) (width 0.2) (layer "F.Cu") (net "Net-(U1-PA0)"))
 (segment (start 140.815 71.815) (end 144.415 75.415) (width 0.2) (layer "F.Cu") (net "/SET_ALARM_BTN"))
 (segment (start 144.415 77.075) (end 150.915 77.075) (width 0.2) (layer "F.Cu") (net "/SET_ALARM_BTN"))
 (segment (start 140.815 71.095) (end 140.815 71.815) (width 0.2) (layer "F.Cu") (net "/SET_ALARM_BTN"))
 (segment (start 144.415 75.415) (end 144.415 77.075) (width 0.2) (layer "F.Cu") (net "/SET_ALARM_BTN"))
 (segment (start 142.715 80.870836) (end 143.910836 79.675) (width 0.2) (layer "F.Cu") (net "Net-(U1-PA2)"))
 (segment (start 143.910836 79.675) (end 148 79.675) (width 0.2) (layer "F.Cu") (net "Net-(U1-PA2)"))
 (segment (start 141.915 74.735) (end 141.915 83.125) (width 0.2) (layer "F.Cu") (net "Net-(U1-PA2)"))
 (segment (start 141.915 83.125) (end 144.415 85.625) (width 0.2) (layer "F.Cu") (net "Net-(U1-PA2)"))
 (segment (start 140.815 73.635) (end 141.915 74.735) (width 0.2) (layer "F.Cu") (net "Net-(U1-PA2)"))
 (segment (start 144.415 85.625) (end 142.715 83.925) (width 0.2) (layer "F.Cu") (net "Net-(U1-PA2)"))
 (segment (start 142.715 83.925) (end 142.715 80.870836) (width 0.2) (layer "F.Cu") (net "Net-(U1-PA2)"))
 (via (at 148 79.675) (size 0.6) (drill 0.3) (layers "F.Cu" "B.Cu") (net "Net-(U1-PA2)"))
 (segment (start 148 79.675) (end 148 82.71) (width 0.2) (layer "B.Cu") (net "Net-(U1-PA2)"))
 (segment (start 148 82.71) (end 150.915 85.625) (width 0.2) (layer "B.Cu") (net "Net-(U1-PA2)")))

